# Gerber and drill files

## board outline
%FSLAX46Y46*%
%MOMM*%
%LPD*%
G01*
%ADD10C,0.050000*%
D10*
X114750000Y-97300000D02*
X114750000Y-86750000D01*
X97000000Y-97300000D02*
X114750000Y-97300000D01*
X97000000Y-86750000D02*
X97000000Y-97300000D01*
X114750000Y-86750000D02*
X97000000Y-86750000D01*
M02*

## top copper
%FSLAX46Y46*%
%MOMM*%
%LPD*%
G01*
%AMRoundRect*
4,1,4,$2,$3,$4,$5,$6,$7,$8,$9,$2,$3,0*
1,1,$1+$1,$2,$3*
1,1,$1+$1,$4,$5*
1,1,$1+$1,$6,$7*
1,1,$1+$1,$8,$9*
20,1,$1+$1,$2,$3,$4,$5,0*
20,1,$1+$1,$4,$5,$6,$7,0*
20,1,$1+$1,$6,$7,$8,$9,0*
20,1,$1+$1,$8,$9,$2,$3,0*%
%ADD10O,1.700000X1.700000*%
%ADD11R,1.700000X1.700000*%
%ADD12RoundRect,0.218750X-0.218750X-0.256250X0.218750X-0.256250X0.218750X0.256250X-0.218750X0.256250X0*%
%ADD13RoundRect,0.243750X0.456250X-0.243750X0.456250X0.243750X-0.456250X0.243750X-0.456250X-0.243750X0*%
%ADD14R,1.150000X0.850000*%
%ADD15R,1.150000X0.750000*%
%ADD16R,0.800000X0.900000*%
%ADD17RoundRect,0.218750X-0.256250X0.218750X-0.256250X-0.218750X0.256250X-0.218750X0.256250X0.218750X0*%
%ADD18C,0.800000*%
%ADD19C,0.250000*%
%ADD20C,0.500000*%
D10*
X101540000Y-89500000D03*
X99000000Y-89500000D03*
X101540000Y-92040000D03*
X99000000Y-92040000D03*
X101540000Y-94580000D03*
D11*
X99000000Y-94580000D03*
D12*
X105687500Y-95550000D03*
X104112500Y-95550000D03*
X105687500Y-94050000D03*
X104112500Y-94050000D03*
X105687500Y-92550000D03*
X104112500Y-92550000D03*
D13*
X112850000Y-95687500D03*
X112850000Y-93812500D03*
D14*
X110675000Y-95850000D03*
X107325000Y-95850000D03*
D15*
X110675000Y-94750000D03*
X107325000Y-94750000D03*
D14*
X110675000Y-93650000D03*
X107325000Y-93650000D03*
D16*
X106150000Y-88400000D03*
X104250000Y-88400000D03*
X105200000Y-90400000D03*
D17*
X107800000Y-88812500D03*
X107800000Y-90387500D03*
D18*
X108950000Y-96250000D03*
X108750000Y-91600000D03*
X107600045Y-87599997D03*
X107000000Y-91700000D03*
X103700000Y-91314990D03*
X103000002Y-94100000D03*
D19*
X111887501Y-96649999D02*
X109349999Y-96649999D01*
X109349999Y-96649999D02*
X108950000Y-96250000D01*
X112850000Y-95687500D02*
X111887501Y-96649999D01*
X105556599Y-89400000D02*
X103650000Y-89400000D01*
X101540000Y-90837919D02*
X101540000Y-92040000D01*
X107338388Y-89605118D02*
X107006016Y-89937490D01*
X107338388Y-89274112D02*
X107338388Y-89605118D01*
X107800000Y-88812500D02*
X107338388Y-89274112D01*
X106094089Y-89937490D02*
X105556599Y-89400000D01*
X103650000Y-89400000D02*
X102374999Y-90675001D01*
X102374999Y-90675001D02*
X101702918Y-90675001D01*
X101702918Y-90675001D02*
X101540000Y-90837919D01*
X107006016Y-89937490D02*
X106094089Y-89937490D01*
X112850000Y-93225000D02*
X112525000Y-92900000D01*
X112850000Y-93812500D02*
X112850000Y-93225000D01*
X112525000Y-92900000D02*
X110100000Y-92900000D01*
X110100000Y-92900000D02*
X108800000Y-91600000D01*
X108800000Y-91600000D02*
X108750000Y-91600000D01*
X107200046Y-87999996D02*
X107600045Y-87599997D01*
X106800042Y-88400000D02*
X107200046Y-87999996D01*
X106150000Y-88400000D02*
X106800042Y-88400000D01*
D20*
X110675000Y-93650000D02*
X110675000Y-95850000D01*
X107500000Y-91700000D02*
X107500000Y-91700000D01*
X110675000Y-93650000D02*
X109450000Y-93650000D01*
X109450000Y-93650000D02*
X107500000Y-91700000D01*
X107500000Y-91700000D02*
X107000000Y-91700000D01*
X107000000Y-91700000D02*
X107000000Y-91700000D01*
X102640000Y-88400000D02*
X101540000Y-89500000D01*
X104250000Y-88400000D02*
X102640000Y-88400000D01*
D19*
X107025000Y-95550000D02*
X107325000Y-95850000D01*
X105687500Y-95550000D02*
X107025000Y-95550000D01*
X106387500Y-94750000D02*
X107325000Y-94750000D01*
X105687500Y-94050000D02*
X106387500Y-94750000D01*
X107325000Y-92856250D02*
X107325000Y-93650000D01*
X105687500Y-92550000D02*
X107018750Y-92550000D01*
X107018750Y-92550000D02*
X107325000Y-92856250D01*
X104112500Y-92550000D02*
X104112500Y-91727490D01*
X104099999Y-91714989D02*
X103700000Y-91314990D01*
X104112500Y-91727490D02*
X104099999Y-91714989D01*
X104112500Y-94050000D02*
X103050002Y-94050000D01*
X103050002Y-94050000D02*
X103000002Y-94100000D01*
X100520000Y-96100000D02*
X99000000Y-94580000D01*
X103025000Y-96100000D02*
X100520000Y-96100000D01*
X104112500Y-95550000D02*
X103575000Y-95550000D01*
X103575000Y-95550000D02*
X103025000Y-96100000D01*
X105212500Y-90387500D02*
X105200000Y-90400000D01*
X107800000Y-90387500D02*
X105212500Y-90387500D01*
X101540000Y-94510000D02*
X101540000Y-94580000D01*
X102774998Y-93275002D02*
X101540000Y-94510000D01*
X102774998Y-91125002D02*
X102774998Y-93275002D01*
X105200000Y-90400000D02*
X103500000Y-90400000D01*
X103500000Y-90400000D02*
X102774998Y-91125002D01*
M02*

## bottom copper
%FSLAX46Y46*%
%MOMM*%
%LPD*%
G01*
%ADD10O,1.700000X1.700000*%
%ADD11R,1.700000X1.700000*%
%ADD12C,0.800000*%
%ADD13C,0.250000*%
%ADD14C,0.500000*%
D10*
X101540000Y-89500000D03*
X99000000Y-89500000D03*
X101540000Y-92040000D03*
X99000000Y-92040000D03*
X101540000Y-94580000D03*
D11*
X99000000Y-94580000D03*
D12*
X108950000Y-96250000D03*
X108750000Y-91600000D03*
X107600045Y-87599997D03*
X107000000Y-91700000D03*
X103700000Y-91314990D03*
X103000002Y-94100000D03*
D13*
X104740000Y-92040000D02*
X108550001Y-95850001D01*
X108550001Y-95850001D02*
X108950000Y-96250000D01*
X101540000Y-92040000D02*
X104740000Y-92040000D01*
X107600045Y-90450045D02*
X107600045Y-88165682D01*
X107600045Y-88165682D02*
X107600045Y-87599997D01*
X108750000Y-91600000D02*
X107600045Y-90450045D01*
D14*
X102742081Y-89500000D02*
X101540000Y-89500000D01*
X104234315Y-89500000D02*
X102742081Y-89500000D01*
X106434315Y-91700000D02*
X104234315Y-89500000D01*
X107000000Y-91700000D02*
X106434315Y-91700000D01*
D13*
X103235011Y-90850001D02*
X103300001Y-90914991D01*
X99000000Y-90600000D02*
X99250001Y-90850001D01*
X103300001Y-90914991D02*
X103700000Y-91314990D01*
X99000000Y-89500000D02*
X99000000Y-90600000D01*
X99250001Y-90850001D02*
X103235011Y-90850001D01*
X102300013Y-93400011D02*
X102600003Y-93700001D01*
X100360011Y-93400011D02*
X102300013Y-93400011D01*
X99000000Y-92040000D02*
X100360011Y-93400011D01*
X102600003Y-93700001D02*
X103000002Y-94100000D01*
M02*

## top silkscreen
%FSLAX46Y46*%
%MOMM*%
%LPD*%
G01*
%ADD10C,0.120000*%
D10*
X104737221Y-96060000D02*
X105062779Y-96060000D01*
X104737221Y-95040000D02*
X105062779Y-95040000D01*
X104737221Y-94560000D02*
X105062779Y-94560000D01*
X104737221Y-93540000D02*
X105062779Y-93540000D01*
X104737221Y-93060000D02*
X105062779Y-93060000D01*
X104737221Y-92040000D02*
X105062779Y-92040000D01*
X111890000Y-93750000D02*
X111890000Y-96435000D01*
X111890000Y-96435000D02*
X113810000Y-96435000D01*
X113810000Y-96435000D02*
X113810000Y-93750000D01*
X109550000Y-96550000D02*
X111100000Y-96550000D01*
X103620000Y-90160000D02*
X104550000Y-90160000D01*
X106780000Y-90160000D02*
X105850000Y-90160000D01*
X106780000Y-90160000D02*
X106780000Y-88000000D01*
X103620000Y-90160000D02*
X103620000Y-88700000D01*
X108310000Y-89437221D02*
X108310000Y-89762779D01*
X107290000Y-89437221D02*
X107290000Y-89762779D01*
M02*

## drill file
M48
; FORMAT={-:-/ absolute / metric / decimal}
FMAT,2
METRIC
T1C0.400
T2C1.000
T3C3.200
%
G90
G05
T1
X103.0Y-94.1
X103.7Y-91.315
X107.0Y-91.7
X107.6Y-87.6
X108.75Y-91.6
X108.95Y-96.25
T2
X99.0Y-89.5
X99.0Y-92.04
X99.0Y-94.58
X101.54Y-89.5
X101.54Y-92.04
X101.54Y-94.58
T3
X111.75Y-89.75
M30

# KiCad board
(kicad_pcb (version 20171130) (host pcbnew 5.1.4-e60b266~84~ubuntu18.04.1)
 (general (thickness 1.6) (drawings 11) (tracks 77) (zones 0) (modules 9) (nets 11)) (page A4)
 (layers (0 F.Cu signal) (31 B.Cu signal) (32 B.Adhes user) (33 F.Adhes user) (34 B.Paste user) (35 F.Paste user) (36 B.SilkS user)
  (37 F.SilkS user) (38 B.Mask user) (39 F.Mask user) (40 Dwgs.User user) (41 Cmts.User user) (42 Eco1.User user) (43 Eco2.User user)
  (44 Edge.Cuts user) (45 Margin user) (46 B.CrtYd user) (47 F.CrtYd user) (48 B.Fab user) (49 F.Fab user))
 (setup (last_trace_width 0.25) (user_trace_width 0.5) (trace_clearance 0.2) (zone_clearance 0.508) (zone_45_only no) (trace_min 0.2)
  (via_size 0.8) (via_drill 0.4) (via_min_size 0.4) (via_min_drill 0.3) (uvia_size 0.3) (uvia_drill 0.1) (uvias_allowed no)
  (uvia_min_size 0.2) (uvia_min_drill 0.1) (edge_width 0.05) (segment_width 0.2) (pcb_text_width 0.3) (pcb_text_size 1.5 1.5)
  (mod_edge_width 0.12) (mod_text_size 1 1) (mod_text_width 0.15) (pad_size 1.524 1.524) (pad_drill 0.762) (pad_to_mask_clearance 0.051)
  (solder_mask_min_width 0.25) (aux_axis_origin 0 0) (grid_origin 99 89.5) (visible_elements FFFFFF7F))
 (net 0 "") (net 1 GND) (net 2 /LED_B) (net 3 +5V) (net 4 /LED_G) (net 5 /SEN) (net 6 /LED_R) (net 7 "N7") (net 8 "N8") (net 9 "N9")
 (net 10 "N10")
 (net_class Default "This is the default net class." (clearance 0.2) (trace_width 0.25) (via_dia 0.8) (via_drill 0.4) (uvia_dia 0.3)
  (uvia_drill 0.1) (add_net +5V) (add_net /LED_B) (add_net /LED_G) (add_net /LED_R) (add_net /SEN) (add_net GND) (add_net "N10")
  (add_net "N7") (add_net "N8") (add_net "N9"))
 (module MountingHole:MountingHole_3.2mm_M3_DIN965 (layer F.Cu) (at 111.75 89.75)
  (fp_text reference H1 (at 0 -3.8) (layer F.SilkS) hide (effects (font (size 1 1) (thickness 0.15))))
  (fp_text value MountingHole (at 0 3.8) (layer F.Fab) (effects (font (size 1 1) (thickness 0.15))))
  (pad 1 np_thru_hole circle (at 0 0) (size 3.2 3.2) (drill 3.2) (layers *.Cu *.Mask)))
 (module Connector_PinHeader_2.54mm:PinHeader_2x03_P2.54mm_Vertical (layer B.Cu) (at 99 94.58)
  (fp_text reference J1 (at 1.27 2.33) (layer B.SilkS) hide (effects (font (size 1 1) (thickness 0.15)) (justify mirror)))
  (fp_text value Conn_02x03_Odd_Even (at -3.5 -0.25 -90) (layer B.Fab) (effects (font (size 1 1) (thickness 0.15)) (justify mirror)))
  (pad 6 thru_hole oval (at 2.54 -5.08) (size 1.7 1.7) (drill 1) (layers *.Cu *.Mask) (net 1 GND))
  (pad 5 thru_hole oval (at 0 -5.08) (size 1.7 1.7) (drill 1) (layers *.Cu *.Mask) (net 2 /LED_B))
  (pad 4 thru_hole oval (at 2.54 -2.54) (size 1.7 1.7) (drill 1) (layers *.Cu *.Mask) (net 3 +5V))
  (pad 3 thru_hole oval (at 0 -2.54) (size 1.7 1.7) (drill 1) (layers *.Cu *.Mask) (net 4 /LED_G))
  (pad 2 thru_hole oval (at 2.54 0) (size 1.7 1.7) (drill 1) (layers *.Cu *.Mask) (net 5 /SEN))
  (pad 1 thru_hole rect (at 0 0) (size 1.7 1.7) (drill 1) (layers *.Cu *.Mask) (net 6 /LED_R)))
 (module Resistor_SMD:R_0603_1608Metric (layer F.Cu) (at 104.9 95.55)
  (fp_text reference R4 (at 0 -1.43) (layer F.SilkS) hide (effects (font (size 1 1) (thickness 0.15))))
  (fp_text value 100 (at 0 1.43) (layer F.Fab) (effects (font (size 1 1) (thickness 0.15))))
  (fp_line (start -0.162779 0.51) (end 0.162779 0.51) (layer F.SilkS) (width 0.12))
  (fp_line (start -0.162779 -0.51) (end 0.162779 -0.51) (layer F.SilkS) (width 0.12))
  (pad 2 smd roundrect (at 0.7875 0) (size 0.875 0.95) (layers F.Cu F.Paste F.Mask) (roundrect_rratio 0.25) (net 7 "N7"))
  (pad 1 smd roundrect (at -0.7875 0) (size 0.875 0.95) (layers F.Cu F.Paste F.Mask) (roundrect_rratio 0.25) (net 6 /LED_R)))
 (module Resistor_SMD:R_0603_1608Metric (layer F.Cu) (at 104.9 94.05)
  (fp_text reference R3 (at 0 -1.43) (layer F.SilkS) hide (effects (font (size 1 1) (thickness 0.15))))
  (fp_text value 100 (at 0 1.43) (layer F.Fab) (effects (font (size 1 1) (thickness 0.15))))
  (fp_line (start -0.162779 0.51) (end 0.162779 0.51) (layer F.SilkS) (width 0.12))
  (fp_line (start -0.162779 -0.51) (end 0.162779 -0.51) (layer F.SilkS) (width 0.12))
  (pad 2 smd roundrect (at 0.7875 0) (size 0.875 0.95) (layers F.Cu F.Paste F.Mask) (roundrect_rratio 0.25) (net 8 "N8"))
  (pad 1 smd roundrect (at -0.7875 0) (size 0.875 0.95) (layers F.Cu F.Paste F.Mask) (roundrect_rratio 0.25) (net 4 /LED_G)))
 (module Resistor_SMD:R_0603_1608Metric (layer F.Cu) (at 104.9 92.55)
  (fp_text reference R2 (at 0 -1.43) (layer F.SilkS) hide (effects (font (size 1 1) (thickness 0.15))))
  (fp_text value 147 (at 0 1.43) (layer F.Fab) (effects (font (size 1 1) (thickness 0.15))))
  (fp_line (start -0.162779 0.51) (end 0.162779 0.51) (layer F.SilkS) (width 0.12))
  (fp_line (start -0.162779 -0.51) (end 0.162779 -0.51) (layer F.SilkS) (width 0.12))
  (pad 2 smd roundrect (at 0.7875 0) (size 0.875 0.95) (layers F.Cu F.Paste F.Mask) (roundrect_rratio 0.25) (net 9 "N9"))
  (pad 1 smd roundrect (at -0.7875 0) (size 0.875 0.95) (layers F.Cu F.Paste F.Mask) (roundrect_rratio 0.25) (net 2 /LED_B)))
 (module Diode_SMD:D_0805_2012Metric (layer F.Cu) (at 112.85 94.75 90)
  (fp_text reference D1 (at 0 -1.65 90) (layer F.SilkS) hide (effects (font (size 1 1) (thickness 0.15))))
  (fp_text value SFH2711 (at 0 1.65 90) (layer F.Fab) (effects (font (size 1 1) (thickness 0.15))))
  (fp_line (start 1 -0.96) (end -1.685 -0.96) (layer F.SilkS) (width 0.12))
  (fp_line (start -1.685 -0.96) (end -1.685 0.96) (layer F.SilkS) (width 0.12))
  (fp_line (start -1.685 0.96) (end 1 0.96) (layer F.SilkS) (width 0.12))
  (pad 1 smd roundrect (at -0.9375 0 90) (size 0.975 1.4) (layers F.Cu F.Paste F.Mask) (roundrect_rratio 0.25) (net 3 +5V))
  (pad 2 smd roundrect (at 0.9375 0 90) (size 0.975 1.4) (layers F.Cu F.Paste F.Mask) (roundrect_rratio 0.25) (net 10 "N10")))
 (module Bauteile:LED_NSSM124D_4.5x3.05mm (layer F.Cu) (at 109 94.75 180)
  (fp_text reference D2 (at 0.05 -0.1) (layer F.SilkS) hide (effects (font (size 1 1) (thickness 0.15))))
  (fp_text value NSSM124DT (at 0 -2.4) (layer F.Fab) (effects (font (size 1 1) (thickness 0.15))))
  (fp_line (start -0.55 -1.8) (end -2.1 -1.8) (layer F.SilkS) (width 0.12))
  (pad 3 smd rect (at -1.675 -1.1 180) (size 1.15 0.85) (layers F.Cu F.Paste F.Mask) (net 1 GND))
  (pad 4 smd rect (at 1.675 -1.1 180) (size 1.15 0.85) (layers F.Cu F.Paste F.Mask) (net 7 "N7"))
  (pad 2 smd rect (at -1.675 0 180) (size 1.15 0.75) (layers F.Cu F.Paste F.Mask) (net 1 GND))
  (pad 5 smd rect (at 1.675 0 180) (size 1.15 0.75) (layers F.Cu F.Paste F.Mask) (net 8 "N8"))
  (pad 1 smd rect (at -1.675 1.1 180) (size 1.15 0.85) (layers F.Cu F.Paste F.Mask) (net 1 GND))
  (pad 6 smd rect (at 1.675 1.1 180) (size 1.15 0.85) (layers F.Cu F.Paste F.Mask) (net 9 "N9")))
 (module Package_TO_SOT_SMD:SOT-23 (layer F.Cu) (at 105.2 89.4 270)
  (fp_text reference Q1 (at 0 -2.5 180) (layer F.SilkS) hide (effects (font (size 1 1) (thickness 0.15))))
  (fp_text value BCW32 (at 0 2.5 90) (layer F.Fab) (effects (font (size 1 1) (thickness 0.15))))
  (fp_line (start 0.76 1.58) (end 0.76 0.65) (layer F.SilkS) (width 0.12))
  (fp_line (start 0.76 -1.58) (end 0.76 -0.65) (layer F.SilkS) (width 0.12))
  (fp_line (start 0.76 -1.58) (end -1.4 -1.58) (layer F.SilkS) (width 0.12))
  (fp_line (start 0.76 1.58) (end -0.7 1.58) (layer F.SilkS) (width 0.12))
  (pad 1 smd rect (at -1 -0.95 270) (size 0.9 0.8) (layers F.Cu F.Paste F.Mask) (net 10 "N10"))
  (pad 2 smd rect (at -1 0.95 270) (size 0.9 0.8) (layers F.Cu F.Paste F.Mask) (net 1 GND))
  (pad 3 smd rect (at 1 0 270) (size 0.9 0.8) (layers F.Cu F.Paste F.Mask) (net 5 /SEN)))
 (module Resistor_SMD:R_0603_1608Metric (layer F.Cu) (at 107.8 89.6 270)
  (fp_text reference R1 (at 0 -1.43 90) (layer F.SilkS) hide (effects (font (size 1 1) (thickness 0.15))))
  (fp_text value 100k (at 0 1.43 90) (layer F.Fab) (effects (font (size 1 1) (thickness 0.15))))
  (fp_line (start -0.162779 -0.51) (end 0.162779 -0.51) (layer F.SilkS) (width 0.12))
  (fp_line (start -0.162779 0.51) (end 0.162779 0.51) (layer F.SilkS) (width 0.12))
  (pad 1 smd roundrect (at -0.7875 0 270) (size 0.875 0.95) (layers F.Cu F.Paste F.Mask) (roundrect_rratio 0.25) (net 3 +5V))
  (pad 2 smd roundrect (at 0.7875 0 270) (size 0.875 0.95) (layers F.Cu F.Paste F.Mask) (roundrect_rratio 0.25) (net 5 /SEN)))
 (gr_line (start 114.75 97.3) (end 114.75 86.75) (layer Edge.Cuts) (width 0.05))
 (gr_line (start 97 97.3) (end 114.75 97.3) (layer Edge.Cuts) (width 0.05))
 (gr_line (start 97 86.75) (end 97 97.3) (layer Edge.Cuts) (width 0.05))
 (gr_line (start 114.75 86.75) (end 97 86.75) (layer Edge.Cuts) (width 0.05))
 (segment (start 104.74 92.04) (end 108.550001 95.850001) (width 0.25) (layer B.Cu) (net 3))
 (segment (start 111.887501 96.649999) (end 109.349999 96.649999) (width 0.25) (layer F.Cu) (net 3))
 (segment (start 108.550001 95.850001) (end 108.95 96.25) (width 0.25) (layer B.Cu) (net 3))
 (via (at 108.95 96.25) (size 0.8) (drill 0.4) (layers F.Cu B.Cu) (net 3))
 (segment (start 109.349999 96.649999) (end 108.95 96.25) (width 0.25) (layer F.Cu) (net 3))
 (segment (start 101.54 92.04) (end 104.74 92.04) (width 0.25) (layer B.Cu) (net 3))
 (segment (start 112.85 95.6875) (end 111.887501 96.649999) (width 0.25) (layer F.Cu) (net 3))
 (segment (start 105.556599 89.4) (end 103.65 89.4) (width 0.25) (layer F.Cu) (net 3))
 (segment (start 101.54 90.837919) (end 101.54 92.04) (width 0.25) (layer F.Cu) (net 3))
 (segment (start 107.338388 89.605118) (end 107.006016 89.93749) (width 0.25) (layer F.Cu) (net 3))
 (segment (start 107.338388 89.274112) (end 107.338388 89.605118) (width 0.25) (layer F.Cu) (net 3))
 (segment (start 107.8 88.8125) (end 107.338388 89.274112) (width 0.25) (layer F.Cu) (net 3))
 (segment (start 106.094089 89.93749) (end 105.556599 89.4) (width 0.25) (layer F.Cu) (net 3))
 (segment (start 103.65 89.4) (end 102.374999 90.675001) (width 0.25) (layer F.Cu) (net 3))
 (segment (start 102.374999 90.675001) (end 101.702918 90.675001) (width 0.25) (layer F.Cu) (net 3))
 (segment (start 101.702918 90.675001) (end 101.54 90.837919) (width 0.25) (layer F.Cu) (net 3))
 (segment (start 107.006016 89.93749) (end 106.094089 89.93749) (width 0.25) (layer F.Cu) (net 3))
 (segment (start 112.85 93.225) (end 112.525 92.9) (width 0.25) (layer F.Cu) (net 10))
 (segment (start 112.85 93.8125) (end 112.85 93.225) (width 0.25) (layer F.Cu) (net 10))
 (segment (start 112.525 92.9) (end 110.1 92.9) (width 0.25) (layer F.Cu) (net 10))
 (via (at 108.75 91.6) (size 0.8) (drill 0.4) (layers F.Cu B.Cu) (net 10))
 (segment (start 110.1 92.9) (end 108.8 91.6) (width 0.25) (layer F.Cu) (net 10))
 (segment (start 108.8 91.6) (end 108.75 91.6) (width 0.25) (layer F.Cu) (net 10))
 (segment (start 107.600045 90.450045) (end 107.600045 88.165682) (width 0.25) (layer B.Cu) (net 10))
 (segment (start 107.600045 88.165682) (end 107.600045 87.599997) (width 0.25) (layer B.Cu) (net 10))
 (segment (start 107.200046 87.999996) (end 107.600045 87.599997) (width 0.25) (layer F.Cu) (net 10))
 (via (at 107.600045 87.599997) (size 0.8) (drill 0.4) (layers F.Cu B.Cu) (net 10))
 (segment (start 108.75 91.6) (end 107.600045 90.450045) (width 0.25) (layer B.Cu) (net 10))
 (segment (start 106.800042 88.4) (end 107.200046 87.999996) (width 0.25) (layer F.Cu) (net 10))
 (segment (start 106.15 88.4) (end 106.800042 88.4) (width 0.25) (layer F.Cu) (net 10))
 (segment (start 110.675 93.65) (end 110.675 95.85) (width 0.5) (layer F.Cu) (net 1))
 (segment (start 107.5 91.7) (end 107.5 91.7) (width 0.5) (layer F.Cu) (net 1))
 (segment (start 110.675 93.65) (end 109.45 93.65) (width 0.5) (layer F.Cu) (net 1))
 (segment (start 109.45 93.65) (end 107.5 91.7) (width 0.5) (layer F.Cu) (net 1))
 (segment (start 107.5 91.7) (end 107 91.7) (width 0.5) (layer F.Cu) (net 1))
 (segment (start 107 91.7) (end 107 91.7) (width 0.5) (layer F.Cu) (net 1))
 (via (at 107 91.7) (size 0.8) (drill 0.4) (layers F.Cu B.Cu) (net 1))
 (segment (start 102.64 88.4) (end 101.54 89.5) (width 0.5) (layer F.Cu) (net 1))
 (segment (start 104.25 88.4) (end 102.64 88.4) (width 0.5) (layer F.Cu) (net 1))
 (segment (start 102.742081 89.5) (end 101.54 89.5) (width 0.5) (layer B.Cu) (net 1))
 (segment (start 104.234315 89.5) (end 102.742081 89.5) (width 0.5) (layer B.Cu) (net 1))
 (segment (start 106.434315 91.7) (end 104.234315 89.5) (width 0.5) (layer B.Cu) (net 1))
 (segment (start 107 91.7) (end 106.434315 91.7) (width 0.5) (layer B.Cu) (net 1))
 (segment (start 107.025 95.55) (end 107.325 95.85) (width 0.25) (layer F.Cu) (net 7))
 (segment (start 105.6875 95.55) (end 107.025 95.55) (width 0.25) (layer F.Cu) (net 7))
 (segment (start 106.3875 94.75) (end 107.325 94.75) (width 0.25) (layer F.Cu) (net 8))
 (segment (start 105.6875 94.05) (end 106.3875 94.75) (width 0.25) (layer F.Cu) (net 8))
 (segment (start 107.325 92.85625) (end 107.325 93.65) (width 0.25) (layer F.Cu) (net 9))
 (segment (start 105.6875 92.55) (end 107.01875 92.55) (width 0.25) (layer F.Cu) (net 9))
 (segment (start 107.01875 92.55) (end 107.325 92.85625) (width 0.25) (layer F.Cu) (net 9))
 (segment (start 103.235011 90.850001) (end 103.300001 90.914991) (width 0.25) (layer B.Cu) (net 2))
 (segment (start 104.1125 92.55) (end 104.1125 91.72749) (width 0.25) (layer F.Cu) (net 2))
 (segment (start 99 90.6) (end 99.250001 90.850001) (width 0.25) (layer B.Cu) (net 2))
 (segment (start 104.099999 91.714989) (end 103.7 91.31499) (width 0.25) (layer F.Cu) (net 2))
 (segment (start 103.300001 90.914991) (end 103.7 91.31499) (width 0.25) (layer B.Cu) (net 2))
 (segment (start 99 89.5) (end 99 90.6) (width 0.25) (layer B.Cu) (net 2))
 (via (at 103.7 91.31499) (size 0.8) (drill 0.4) (layers F.Cu B.Cu) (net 2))
 (segment (start 99.250001 90.850001) (end 103.235011 90.850001) (width 0.25) (layer B.Cu) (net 2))
 (segment (start 104.1125 91.72749) (end 104.099999 91.714989) (width 0.25) (layer F.Cu) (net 2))
 (via (at 103.000002 94.1) (size 0.8) (drill 0.4) (layers F.Cu B.Cu) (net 4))
 (segment (start 104.1125 94.05) (end 103.050002 94.05) (width 0.25) (layer F.Cu) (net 4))
 (segment (start 103.050002 94.05) (end 103.000002 94.1) (width 0.25) (layer F.Cu) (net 4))
 (segment (start 102.300013 93.400011) (end 102.600003 93.700001) (width 0.25) (layer B.Cu) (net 4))
 (segment (start 100.360011 93.400011) (end 102.300013 93.400011) (width 0.25) (layer B.Cu) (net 4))
 (segment (start 99 92.04) (end 100.360011 93.400011) (width 0.25) (layer B.Cu) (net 4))
 (segment (start 102.600003 93.700001) (end 103.000002 94.1) (width 0.25) (layer B.Cu) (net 4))
 (segment (start 100.52 96.1) (end 99 94.58) (width 0.25) (layer F.Cu) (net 6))
 (segment (start 103.025 96.1) (end 100.52 96.1) (width 0.25) (layer F.Cu) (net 6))
 (segment (start 104.1125 95.55) (end 103.575 95.55) (width 0.25) (layer F.Cu) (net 6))
 (segment (start 103.575 95.55) (end 103.025 96.1) (width 0.25) (layer F.Cu) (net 6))
 (segment (start 105.2125 90.3875) (end 105.2 90.4) (width 0.25) (layer F.Cu) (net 5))
 (segment (start 107.8 90.3875) (end 105.2125 90.3875) (width 0.25) (layer F.Cu) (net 5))
 (segment (start 101.54 94.51) (end 101.54 94.58) (width 0.25) (layer F.Cu) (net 5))
 (segment (start 102.774998 93.275002) (end 101.54 94.51) (width 0.25) (layer F.Cu) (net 5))
 (segment (start 102.774998 91.125002) (end 102.774998 93.275002) (width 0.25) (layer F.Cu) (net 5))
 (segment (start 105.2 90.4) (end 103.5 90.4) (width 0.25) (layer F.Cu) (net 5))
 (segment (start 103.5 90.4) (end 102.774998 91.125002) (width 0.25) (layer F.Cu) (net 5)))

